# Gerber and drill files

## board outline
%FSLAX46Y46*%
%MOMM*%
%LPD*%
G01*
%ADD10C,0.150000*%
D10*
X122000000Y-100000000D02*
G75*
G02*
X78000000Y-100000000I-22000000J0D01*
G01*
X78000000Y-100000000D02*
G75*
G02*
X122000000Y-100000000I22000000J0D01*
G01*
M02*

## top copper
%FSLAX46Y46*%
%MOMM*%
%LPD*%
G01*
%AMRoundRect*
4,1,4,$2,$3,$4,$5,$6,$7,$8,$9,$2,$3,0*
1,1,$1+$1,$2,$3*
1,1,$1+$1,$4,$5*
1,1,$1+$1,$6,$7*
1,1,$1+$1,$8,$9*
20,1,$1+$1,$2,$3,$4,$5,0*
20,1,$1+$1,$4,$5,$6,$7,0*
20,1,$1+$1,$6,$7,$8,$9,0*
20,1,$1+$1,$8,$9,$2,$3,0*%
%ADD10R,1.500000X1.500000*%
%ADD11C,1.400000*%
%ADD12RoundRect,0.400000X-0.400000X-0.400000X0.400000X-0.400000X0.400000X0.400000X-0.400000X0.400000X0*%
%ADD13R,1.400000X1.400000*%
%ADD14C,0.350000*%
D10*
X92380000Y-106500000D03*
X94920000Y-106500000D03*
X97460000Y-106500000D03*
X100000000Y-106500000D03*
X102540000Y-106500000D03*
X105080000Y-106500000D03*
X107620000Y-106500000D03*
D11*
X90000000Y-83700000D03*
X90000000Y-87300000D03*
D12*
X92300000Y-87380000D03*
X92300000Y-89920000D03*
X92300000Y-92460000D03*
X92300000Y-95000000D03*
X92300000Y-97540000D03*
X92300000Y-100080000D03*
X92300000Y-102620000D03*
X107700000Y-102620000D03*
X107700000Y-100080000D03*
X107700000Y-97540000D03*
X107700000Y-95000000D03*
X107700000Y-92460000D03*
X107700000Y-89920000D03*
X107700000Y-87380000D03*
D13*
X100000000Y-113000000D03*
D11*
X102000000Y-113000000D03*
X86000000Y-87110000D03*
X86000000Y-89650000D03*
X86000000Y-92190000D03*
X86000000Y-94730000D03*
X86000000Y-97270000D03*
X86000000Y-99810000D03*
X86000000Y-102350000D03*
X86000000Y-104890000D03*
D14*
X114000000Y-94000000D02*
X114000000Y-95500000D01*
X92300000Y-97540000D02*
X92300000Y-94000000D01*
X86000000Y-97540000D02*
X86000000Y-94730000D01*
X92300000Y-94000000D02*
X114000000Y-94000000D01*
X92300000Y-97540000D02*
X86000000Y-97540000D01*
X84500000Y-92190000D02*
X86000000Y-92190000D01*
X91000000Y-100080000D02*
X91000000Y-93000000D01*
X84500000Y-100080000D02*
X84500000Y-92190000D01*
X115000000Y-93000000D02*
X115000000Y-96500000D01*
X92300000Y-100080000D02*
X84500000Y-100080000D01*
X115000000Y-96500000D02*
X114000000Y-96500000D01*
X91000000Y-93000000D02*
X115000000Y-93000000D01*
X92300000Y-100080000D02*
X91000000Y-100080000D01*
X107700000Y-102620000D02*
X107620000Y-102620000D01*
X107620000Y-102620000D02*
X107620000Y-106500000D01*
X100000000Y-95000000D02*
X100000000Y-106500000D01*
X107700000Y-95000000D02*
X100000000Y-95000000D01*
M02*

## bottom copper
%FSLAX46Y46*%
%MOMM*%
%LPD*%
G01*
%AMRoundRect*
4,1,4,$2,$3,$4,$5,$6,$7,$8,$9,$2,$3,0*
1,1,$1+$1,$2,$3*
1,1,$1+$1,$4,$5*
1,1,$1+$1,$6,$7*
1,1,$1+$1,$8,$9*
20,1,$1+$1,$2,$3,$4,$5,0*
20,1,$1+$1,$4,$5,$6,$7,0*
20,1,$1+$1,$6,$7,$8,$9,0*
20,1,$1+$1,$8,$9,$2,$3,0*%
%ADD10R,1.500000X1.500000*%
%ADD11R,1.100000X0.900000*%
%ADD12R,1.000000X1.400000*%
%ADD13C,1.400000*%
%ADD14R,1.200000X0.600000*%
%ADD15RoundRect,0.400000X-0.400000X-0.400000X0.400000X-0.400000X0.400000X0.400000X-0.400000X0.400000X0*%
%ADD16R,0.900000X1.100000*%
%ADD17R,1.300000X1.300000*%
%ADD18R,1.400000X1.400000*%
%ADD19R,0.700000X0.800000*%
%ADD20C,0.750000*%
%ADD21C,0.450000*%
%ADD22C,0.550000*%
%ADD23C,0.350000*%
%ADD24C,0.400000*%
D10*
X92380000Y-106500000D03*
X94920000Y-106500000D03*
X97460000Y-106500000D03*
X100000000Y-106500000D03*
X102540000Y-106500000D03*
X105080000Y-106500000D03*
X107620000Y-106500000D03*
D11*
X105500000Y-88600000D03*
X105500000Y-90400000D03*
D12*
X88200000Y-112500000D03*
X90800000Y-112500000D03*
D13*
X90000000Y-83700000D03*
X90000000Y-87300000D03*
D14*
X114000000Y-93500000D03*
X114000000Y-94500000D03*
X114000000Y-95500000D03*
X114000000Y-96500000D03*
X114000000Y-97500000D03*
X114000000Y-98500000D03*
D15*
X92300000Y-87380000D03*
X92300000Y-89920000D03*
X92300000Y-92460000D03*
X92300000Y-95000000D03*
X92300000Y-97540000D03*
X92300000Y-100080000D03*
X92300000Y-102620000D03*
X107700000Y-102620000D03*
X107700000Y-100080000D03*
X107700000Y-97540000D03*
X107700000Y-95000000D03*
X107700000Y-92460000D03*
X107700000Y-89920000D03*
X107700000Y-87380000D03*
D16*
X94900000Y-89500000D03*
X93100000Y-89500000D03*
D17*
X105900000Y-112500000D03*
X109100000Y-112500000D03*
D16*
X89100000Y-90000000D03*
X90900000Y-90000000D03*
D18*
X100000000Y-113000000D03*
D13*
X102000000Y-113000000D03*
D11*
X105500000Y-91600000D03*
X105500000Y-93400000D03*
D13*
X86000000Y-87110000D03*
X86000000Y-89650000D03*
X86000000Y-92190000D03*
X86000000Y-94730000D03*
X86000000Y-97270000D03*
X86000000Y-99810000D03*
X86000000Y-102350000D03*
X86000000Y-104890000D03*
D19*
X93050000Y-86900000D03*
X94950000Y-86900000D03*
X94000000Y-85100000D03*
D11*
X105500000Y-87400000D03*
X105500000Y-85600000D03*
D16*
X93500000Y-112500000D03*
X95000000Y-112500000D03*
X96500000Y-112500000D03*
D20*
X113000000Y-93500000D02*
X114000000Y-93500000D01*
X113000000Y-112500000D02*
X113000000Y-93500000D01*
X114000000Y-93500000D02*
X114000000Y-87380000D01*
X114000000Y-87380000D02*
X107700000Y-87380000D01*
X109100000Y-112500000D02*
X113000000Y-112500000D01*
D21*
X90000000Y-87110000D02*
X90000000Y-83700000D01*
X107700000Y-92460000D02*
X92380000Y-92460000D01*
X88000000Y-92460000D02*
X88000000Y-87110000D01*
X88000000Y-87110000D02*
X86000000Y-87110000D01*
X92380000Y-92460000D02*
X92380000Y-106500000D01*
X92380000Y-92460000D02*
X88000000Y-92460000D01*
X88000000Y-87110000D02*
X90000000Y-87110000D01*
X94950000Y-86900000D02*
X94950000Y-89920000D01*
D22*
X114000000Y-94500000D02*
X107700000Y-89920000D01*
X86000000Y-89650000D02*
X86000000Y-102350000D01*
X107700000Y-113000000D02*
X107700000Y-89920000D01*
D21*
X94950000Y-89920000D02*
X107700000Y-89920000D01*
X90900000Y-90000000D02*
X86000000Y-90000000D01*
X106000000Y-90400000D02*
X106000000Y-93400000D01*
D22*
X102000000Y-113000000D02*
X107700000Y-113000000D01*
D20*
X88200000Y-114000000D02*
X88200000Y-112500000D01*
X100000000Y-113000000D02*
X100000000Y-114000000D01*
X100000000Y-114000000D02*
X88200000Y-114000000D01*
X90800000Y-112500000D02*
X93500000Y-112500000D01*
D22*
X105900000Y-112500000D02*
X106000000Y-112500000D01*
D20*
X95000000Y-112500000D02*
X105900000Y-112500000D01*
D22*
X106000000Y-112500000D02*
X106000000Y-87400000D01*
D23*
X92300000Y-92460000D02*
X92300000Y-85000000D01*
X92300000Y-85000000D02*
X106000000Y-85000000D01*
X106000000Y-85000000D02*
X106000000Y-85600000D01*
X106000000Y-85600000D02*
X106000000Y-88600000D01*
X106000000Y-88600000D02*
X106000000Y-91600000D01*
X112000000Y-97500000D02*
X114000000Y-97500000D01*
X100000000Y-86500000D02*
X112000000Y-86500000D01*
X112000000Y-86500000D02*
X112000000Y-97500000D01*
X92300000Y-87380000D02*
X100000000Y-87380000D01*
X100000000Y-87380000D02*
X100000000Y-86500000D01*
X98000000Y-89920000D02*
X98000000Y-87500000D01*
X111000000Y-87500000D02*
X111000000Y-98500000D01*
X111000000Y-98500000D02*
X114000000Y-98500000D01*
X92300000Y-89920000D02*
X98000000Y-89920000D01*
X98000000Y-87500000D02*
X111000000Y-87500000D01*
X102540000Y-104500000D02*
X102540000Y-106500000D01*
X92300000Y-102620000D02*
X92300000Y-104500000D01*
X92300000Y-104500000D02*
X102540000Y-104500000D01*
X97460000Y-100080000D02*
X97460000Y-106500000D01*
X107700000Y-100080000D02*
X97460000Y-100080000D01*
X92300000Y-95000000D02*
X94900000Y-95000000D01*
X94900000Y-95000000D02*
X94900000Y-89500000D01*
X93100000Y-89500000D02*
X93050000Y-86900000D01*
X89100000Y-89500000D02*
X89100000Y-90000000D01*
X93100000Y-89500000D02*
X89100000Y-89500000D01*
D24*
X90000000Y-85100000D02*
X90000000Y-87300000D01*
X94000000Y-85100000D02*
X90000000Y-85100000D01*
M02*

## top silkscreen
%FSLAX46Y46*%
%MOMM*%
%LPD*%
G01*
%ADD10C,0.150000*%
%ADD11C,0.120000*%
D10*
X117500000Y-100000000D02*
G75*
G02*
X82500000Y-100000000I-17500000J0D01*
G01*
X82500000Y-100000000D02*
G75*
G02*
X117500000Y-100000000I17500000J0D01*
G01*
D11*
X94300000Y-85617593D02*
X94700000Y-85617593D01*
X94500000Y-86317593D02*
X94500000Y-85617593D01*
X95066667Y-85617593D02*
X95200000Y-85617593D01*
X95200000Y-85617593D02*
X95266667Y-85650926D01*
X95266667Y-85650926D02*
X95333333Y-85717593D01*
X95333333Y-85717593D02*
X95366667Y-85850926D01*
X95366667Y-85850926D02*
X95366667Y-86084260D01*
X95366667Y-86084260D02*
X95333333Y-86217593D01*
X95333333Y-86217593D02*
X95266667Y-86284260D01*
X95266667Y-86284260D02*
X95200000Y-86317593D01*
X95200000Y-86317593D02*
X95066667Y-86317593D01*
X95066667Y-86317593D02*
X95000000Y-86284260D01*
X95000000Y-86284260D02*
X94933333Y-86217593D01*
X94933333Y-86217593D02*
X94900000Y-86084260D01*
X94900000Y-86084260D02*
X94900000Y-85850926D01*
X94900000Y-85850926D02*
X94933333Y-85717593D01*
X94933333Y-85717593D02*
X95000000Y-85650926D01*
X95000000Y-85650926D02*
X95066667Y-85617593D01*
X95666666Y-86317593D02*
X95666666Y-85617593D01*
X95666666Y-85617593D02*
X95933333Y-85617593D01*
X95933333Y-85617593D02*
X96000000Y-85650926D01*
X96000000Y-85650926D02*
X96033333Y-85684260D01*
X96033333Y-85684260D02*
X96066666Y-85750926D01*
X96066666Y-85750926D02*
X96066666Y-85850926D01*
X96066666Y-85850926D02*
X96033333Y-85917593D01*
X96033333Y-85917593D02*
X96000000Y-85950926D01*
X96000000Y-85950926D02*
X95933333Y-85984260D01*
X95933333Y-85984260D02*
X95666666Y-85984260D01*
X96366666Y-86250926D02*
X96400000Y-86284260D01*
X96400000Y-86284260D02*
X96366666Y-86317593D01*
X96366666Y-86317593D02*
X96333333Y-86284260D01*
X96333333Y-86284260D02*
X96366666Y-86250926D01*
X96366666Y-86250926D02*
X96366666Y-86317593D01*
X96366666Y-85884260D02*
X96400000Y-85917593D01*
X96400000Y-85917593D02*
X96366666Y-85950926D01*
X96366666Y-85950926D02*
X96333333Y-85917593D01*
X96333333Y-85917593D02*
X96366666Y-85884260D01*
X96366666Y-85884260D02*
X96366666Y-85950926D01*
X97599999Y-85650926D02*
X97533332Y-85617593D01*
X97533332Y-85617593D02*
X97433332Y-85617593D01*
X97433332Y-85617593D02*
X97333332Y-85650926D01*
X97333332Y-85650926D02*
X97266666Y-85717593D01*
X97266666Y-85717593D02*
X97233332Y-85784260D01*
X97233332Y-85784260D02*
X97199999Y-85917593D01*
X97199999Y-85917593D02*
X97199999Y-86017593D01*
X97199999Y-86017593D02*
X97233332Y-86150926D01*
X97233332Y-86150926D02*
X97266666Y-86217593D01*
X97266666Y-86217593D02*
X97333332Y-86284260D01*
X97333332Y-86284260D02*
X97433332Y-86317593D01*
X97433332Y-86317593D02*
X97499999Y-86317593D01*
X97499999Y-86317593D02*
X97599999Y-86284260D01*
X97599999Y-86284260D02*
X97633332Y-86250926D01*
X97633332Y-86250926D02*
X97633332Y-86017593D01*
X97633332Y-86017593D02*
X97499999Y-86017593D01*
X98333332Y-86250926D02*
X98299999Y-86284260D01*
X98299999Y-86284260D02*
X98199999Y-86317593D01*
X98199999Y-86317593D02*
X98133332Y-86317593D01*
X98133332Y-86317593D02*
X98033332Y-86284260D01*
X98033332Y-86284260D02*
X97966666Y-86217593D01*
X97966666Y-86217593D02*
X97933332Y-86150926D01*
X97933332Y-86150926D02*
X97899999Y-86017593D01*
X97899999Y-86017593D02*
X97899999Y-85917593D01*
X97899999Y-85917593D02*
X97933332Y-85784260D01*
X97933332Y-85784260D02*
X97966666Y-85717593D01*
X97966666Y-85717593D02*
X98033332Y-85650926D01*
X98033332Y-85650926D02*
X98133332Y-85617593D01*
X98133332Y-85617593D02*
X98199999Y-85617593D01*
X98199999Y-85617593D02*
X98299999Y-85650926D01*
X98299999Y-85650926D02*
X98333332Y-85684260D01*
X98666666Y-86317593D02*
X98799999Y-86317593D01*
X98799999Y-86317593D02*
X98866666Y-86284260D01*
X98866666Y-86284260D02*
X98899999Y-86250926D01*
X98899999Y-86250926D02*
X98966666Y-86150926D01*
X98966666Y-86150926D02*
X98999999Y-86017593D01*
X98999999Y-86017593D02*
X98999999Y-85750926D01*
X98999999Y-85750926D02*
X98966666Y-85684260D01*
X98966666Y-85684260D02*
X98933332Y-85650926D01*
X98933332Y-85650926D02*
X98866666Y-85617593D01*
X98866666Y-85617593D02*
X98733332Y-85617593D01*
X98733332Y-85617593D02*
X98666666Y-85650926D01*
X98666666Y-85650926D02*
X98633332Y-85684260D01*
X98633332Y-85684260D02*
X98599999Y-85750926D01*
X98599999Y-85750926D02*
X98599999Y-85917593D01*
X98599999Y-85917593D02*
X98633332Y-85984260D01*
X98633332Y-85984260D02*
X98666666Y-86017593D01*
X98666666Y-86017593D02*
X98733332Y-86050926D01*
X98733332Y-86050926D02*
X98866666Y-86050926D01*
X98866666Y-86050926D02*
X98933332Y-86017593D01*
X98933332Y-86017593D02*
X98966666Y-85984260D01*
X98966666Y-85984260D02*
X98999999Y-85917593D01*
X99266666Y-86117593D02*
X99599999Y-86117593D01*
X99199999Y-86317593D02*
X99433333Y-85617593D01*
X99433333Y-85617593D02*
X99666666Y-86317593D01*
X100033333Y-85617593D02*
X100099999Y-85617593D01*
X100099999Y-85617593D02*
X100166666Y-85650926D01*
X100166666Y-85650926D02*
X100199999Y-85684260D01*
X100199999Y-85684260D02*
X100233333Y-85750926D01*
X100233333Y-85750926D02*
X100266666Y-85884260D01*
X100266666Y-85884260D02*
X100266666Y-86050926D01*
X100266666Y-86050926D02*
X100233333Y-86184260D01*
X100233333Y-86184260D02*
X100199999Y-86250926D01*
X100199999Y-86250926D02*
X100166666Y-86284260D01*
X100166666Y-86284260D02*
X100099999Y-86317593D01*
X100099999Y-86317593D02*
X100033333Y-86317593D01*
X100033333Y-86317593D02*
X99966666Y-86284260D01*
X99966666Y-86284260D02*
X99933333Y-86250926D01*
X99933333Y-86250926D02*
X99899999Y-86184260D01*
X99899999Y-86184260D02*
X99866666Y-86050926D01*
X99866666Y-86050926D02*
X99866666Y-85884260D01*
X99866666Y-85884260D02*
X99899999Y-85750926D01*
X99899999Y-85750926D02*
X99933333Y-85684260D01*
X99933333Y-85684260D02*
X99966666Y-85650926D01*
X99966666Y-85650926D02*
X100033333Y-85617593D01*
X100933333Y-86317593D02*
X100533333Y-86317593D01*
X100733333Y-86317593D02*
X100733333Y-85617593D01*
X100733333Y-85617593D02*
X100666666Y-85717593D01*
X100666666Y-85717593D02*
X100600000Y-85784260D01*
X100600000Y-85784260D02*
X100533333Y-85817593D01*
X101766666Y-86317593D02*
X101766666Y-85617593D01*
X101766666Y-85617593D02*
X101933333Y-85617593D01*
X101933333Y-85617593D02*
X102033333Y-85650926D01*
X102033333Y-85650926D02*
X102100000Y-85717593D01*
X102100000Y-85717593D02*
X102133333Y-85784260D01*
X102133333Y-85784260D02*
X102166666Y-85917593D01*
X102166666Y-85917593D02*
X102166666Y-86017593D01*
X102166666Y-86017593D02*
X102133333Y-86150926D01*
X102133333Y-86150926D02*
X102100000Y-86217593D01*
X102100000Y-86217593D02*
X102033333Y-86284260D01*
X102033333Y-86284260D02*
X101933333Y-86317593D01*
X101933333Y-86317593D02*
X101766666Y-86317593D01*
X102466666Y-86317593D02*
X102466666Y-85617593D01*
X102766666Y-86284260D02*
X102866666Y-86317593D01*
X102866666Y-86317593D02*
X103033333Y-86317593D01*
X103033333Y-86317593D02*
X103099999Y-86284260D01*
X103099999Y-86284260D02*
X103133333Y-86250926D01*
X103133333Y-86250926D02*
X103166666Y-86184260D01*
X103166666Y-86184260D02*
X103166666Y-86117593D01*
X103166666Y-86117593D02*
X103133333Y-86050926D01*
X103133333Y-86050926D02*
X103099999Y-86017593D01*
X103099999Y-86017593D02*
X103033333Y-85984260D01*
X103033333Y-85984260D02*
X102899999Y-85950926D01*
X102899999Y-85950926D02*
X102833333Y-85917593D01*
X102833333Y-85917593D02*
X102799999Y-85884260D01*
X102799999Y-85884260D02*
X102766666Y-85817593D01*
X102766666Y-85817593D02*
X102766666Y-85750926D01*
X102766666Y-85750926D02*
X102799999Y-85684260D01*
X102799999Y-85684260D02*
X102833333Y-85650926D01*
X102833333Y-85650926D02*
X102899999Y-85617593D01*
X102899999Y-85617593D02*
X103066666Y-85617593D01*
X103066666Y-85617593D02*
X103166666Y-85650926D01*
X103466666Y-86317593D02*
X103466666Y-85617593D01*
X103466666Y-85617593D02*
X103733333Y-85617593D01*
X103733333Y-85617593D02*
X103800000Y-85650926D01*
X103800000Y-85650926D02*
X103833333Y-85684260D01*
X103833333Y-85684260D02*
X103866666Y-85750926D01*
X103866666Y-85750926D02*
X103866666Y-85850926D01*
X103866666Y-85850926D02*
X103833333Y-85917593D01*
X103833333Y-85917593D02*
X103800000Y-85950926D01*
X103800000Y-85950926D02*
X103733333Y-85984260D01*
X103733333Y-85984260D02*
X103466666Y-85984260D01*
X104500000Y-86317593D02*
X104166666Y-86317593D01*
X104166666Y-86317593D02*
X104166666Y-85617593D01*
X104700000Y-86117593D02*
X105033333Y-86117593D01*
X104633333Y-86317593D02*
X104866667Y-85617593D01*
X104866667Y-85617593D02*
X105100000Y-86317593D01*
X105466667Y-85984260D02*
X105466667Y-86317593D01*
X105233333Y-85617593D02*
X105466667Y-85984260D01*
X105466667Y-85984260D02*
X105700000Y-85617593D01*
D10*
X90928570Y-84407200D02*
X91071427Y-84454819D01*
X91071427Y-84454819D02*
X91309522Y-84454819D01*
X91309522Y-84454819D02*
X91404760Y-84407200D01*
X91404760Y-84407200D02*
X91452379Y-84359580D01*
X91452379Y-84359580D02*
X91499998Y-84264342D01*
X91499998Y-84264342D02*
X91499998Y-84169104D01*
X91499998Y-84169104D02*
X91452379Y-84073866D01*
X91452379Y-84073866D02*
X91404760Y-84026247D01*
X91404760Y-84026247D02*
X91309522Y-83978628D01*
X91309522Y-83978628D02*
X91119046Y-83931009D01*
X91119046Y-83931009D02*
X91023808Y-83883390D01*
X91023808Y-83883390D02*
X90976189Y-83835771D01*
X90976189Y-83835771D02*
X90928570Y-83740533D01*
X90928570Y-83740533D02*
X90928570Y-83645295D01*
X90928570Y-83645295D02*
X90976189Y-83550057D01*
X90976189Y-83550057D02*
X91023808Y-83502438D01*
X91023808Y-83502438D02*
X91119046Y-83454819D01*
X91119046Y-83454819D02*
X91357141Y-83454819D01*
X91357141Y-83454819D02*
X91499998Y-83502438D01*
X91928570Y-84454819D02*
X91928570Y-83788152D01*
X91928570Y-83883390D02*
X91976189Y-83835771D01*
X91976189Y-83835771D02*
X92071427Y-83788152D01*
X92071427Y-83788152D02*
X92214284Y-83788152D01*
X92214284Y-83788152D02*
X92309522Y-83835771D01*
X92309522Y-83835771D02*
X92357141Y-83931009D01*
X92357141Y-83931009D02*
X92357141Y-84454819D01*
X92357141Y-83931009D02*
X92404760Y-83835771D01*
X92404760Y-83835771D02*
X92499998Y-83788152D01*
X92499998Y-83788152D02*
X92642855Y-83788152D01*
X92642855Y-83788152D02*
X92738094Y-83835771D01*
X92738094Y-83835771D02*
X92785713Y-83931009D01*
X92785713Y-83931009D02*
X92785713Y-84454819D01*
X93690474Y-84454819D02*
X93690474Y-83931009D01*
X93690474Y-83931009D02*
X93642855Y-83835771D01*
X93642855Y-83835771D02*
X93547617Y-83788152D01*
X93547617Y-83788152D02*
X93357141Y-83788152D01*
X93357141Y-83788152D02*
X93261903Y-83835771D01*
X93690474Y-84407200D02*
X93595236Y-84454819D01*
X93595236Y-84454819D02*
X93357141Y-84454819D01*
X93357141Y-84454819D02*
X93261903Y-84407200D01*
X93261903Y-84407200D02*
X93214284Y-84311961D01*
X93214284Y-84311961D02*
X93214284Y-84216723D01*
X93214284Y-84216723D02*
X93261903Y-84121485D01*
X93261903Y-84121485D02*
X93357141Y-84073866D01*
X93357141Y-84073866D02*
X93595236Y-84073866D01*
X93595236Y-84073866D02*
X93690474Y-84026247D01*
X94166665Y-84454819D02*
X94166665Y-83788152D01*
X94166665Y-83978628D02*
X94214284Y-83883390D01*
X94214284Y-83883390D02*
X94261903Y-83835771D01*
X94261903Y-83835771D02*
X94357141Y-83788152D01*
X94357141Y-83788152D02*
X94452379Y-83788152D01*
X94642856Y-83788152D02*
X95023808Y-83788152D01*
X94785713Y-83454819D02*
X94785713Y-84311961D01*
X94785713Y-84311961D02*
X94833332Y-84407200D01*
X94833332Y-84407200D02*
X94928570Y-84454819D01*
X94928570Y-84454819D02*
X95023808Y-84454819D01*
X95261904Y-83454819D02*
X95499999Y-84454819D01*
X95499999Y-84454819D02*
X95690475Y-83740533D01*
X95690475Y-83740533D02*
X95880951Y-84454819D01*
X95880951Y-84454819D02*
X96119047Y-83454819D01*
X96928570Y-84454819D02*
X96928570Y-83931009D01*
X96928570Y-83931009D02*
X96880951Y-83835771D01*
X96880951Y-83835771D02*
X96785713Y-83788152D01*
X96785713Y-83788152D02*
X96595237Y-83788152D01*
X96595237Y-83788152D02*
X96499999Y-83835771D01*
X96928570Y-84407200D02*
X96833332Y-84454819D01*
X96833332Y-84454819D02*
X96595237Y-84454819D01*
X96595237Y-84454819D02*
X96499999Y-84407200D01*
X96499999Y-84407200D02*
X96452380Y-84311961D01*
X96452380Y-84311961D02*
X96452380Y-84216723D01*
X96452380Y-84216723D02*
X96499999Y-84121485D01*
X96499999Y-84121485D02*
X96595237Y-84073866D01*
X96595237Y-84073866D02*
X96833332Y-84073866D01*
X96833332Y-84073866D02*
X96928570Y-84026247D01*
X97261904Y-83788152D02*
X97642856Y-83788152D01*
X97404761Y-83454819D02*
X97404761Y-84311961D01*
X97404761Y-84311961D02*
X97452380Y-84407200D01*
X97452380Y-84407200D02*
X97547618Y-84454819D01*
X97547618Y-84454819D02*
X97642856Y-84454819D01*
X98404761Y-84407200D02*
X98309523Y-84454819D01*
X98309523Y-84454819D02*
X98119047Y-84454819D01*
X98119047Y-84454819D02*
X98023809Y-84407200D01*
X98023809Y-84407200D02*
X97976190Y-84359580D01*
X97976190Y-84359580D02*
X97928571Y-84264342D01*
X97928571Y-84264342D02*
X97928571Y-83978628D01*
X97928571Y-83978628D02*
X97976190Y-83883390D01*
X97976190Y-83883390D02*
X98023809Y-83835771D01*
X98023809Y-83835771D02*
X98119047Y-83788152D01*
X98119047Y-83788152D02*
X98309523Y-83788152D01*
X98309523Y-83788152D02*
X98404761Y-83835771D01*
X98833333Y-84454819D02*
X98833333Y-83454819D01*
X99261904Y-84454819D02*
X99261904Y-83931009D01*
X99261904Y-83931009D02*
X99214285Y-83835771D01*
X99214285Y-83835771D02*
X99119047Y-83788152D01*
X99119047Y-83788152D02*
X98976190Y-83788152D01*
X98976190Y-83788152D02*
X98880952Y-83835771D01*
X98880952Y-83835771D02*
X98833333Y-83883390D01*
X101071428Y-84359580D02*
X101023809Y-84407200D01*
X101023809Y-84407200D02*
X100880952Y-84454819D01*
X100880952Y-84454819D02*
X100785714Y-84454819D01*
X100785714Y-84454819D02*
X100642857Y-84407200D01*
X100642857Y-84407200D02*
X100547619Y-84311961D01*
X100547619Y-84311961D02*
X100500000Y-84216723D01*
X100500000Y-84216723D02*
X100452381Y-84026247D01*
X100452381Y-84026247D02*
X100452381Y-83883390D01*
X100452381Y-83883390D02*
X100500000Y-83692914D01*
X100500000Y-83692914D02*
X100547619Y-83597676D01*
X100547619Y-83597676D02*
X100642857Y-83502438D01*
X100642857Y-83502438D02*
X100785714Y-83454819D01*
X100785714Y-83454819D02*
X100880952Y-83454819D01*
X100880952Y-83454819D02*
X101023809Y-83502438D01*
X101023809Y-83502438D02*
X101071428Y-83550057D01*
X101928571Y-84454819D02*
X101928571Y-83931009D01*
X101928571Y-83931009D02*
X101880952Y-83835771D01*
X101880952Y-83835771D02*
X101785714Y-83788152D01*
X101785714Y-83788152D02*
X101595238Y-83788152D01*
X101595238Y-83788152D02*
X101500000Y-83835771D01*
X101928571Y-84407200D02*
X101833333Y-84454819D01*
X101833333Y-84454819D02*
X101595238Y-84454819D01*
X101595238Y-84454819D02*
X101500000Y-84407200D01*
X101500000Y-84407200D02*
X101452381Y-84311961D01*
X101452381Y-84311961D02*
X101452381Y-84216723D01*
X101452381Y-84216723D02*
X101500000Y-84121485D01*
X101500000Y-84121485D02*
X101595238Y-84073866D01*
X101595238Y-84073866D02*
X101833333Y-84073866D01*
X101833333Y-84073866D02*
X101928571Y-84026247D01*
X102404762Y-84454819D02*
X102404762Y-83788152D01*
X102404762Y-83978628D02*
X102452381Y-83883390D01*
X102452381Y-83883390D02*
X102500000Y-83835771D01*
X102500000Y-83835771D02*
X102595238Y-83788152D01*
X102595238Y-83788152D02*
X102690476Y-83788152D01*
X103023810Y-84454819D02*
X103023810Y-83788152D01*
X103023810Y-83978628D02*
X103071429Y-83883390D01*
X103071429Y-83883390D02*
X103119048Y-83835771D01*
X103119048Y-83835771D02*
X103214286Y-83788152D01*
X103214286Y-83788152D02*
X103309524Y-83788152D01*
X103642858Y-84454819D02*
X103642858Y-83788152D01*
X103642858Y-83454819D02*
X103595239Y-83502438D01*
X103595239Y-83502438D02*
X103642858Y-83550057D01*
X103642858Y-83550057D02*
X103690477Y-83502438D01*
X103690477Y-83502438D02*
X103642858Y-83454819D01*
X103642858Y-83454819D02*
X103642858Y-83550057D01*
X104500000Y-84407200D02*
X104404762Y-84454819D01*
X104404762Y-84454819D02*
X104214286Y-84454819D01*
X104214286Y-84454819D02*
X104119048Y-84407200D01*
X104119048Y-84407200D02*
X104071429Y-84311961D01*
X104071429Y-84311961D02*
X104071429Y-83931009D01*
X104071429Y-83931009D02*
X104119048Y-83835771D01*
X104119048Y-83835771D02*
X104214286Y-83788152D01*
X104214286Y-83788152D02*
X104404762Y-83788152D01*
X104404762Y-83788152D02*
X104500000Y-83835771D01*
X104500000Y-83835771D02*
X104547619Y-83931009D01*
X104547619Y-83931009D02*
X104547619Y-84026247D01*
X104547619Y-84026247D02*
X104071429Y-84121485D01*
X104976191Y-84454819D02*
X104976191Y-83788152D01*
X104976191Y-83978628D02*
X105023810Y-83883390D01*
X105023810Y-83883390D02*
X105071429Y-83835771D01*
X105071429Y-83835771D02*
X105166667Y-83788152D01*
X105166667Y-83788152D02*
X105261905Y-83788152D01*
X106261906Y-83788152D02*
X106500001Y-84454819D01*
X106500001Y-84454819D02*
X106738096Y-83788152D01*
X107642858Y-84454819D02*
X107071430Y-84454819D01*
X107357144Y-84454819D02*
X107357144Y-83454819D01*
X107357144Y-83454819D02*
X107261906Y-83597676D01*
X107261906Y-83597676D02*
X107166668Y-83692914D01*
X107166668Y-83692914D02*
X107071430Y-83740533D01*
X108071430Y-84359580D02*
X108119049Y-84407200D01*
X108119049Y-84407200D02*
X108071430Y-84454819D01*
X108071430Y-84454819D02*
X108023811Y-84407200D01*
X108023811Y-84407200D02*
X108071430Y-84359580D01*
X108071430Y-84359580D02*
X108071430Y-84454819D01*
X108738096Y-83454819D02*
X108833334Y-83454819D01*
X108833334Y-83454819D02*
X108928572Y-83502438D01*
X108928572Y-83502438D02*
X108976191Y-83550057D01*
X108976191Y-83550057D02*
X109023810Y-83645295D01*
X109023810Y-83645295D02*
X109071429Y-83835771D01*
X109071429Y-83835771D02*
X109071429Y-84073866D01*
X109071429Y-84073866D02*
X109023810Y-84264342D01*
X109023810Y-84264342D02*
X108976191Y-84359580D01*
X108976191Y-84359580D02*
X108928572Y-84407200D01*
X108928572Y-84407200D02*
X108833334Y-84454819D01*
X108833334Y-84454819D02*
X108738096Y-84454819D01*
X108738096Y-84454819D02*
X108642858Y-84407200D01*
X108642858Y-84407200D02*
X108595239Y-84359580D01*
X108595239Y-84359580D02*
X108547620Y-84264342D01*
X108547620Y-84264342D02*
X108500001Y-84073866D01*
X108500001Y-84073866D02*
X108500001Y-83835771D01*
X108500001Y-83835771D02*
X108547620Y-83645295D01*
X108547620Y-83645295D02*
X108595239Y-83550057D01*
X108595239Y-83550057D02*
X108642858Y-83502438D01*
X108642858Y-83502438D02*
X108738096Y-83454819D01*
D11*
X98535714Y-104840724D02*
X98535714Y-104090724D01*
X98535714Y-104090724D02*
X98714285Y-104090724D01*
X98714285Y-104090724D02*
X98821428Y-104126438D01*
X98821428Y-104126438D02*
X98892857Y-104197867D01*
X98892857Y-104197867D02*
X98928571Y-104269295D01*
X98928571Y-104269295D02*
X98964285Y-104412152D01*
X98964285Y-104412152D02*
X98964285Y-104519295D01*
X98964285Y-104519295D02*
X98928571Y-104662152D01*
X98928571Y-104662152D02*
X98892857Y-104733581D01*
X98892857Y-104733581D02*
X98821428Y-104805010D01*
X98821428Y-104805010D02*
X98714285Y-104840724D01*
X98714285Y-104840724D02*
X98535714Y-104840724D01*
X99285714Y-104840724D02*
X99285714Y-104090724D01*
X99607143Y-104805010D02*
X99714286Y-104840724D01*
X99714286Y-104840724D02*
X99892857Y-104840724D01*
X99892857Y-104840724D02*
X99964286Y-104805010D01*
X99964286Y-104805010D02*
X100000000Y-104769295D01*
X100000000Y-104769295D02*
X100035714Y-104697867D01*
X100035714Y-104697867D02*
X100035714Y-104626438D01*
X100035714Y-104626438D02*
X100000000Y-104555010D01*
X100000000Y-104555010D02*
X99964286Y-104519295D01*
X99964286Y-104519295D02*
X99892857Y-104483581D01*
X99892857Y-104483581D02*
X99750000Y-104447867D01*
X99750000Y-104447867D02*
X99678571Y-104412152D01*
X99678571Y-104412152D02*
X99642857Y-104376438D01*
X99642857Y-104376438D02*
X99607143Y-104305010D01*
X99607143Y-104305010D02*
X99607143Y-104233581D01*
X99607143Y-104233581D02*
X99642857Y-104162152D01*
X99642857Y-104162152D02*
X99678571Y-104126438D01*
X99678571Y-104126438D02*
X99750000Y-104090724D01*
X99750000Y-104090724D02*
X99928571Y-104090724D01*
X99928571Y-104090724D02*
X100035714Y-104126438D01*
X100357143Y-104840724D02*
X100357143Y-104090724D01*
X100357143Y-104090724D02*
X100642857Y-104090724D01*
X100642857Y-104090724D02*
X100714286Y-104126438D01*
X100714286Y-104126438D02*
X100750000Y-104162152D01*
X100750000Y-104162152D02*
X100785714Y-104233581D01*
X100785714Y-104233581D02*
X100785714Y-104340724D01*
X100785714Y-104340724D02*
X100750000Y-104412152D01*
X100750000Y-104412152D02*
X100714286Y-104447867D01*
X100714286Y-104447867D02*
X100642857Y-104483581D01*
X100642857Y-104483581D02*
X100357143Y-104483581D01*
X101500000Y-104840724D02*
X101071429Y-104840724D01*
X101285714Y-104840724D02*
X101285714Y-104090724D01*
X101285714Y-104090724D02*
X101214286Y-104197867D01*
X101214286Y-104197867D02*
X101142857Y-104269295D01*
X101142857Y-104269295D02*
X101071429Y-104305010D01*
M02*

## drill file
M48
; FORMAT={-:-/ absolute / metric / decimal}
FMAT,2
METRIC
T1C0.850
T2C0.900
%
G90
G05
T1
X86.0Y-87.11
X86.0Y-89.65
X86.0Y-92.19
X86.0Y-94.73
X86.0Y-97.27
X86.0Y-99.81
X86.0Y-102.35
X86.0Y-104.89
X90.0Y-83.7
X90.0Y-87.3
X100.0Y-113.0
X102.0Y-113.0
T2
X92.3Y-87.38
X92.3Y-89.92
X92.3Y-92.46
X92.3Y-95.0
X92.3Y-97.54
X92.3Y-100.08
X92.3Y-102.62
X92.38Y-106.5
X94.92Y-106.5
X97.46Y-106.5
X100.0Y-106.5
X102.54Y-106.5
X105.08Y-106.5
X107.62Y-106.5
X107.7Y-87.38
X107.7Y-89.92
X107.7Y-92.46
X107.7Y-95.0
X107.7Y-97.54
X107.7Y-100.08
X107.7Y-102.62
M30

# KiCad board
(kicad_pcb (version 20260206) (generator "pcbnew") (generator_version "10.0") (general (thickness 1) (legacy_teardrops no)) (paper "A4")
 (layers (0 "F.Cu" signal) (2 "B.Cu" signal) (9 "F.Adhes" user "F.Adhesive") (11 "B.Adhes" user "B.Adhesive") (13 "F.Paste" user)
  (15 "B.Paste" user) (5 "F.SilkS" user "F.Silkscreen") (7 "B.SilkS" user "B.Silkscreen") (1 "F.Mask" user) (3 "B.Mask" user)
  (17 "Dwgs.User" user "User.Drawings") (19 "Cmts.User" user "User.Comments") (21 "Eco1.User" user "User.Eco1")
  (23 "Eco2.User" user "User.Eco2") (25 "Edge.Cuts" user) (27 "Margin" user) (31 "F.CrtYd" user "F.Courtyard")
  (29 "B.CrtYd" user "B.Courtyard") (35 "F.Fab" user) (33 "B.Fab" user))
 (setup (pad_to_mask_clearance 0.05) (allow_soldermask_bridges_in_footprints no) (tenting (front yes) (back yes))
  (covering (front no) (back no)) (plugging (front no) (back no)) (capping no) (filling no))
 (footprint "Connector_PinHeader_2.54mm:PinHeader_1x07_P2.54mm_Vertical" (layer "F.Cu") (at 100 106.5)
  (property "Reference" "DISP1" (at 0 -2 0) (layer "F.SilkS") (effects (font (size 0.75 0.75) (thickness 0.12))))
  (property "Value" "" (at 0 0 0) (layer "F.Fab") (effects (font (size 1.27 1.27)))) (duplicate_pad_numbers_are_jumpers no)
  (pad "1" thru_hole rect (at -7.62 0) (size 1.5 1.5) (drill 0.9) (layers "*.Cu" "*.Mask") (remove_unused_layers no) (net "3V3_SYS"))
  (pad "2" thru_hole rect (at -5.08 0) (size 1.5 1.5) (drill 0.9) (layers "*.Cu" "*.Mask") (remove_unused_layers no) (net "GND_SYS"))
  (pad "3" thru_hole rect (at -2.54 0) (size 1.5 1.5) (drill 0.9) (layers "*.Cu" "*.Mask") (remove_unused_layers no) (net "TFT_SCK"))
  (pad "4" thru_hole rect (at 0 0) (size 1.5 1.5) (drill 0.9) (layers "*.Cu" "*.Mask") (remove_unused_layers no) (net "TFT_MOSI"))
  (pad "5" thru_hole rect (at 2.54 0) (size 1.5 1.5) (drill 0.9) (layers "*.Cu" "*.Mask") (remove_unused_layers no) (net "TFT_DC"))
  (pad "6" thru_hole rect (at 5.08 0) (size 1.5 1.5) (drill 0.9) (layers "*.Cu" "*.Mask") (remove_unused_layers no) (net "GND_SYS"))
  (pad "7" thru_hole rect (at 7.62 0) (size 1.5 1.5) (drill 0.9) (layers "*.Cu" "*.Mask") (remove_unused_layers no) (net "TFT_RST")))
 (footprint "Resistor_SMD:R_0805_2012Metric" (layer "B.Cu") (at 105.5 89.5)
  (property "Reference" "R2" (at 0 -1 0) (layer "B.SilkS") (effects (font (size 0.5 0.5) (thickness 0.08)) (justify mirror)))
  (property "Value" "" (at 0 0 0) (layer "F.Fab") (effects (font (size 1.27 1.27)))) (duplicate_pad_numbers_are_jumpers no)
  (pad "1" smd rect (at 0 -0.9) (size 1.1 0.9) (layers "B.Cu" "B.Mask" "B.Paste") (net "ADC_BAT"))
  (pad "2" smd rect (at 0 0.9) (size 1.1 0.9) (layers "B.Cu" "B.Mask" "B.Paste") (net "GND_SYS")))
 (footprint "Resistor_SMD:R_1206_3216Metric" (layer "B.Cu") (at 89.5 112.5)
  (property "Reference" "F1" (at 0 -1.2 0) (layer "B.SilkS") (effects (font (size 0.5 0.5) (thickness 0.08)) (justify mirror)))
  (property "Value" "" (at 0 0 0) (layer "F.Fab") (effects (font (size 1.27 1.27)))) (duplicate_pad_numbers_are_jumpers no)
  (pad "1" smd rect (at -1.3 0) (size 1 1.4) (layers "B.Cu" "B.Mask" "B.Paste") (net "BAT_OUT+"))
  (pad "2" smd rect (at 1.3 0) (size 1 1.4) (layers "B.Cu" "B.Mask" "B.Paste") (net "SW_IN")))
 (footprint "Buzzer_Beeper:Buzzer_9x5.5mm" (layer "B.Cu") (at 90 85.5)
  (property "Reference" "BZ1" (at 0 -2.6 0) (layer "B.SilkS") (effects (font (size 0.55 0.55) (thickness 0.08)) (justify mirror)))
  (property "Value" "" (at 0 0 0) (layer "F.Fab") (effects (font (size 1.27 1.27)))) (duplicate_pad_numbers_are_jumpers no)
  (pad "1" thru_hole circle (at 0 -1.8) (size 1.4 1.4) (drill 0.85) (layers "*.Cu" "*.Mask") (remove_unused_layers no) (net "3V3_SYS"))
  (pad "2" thru_hole circle (at 0 1.8) (size 1.4 1.4) (drill 0.85) (layers "*.Cu" "*.Mask") (remove_unused_layers no) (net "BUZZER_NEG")))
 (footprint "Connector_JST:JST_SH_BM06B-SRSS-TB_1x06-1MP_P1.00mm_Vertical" (layer "B.Cu") (at 114 96)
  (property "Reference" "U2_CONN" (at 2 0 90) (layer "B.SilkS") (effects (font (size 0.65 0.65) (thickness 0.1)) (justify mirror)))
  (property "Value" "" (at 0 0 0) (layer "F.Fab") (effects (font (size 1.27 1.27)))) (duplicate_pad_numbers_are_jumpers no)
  (pad "1" smd rect (at 0 -2.5) (size 1.2 0.6) (layers "B.Cu" "B.Mask" "B.Paste") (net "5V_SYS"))
  (pad "2" smd rect (at 0 -1.5) (size 1.2 0.6) (layers "B.Cu" "B.Mask" "B.Paste") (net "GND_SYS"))
  (pad "3" smd rect (at 0 -0.5) (size 1.2 0.6) (layers "B.Cu" "B.Mask" "B.Paste") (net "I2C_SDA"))
  (pad "4" smd rect (at 0 0.5) (size 1.2 0.6) (layers "B.Cu" "B.Mask" "B.Paste") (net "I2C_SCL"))
  (pad "5" smd rect (at 0 1.5) (size 1.2 0.6) (layers "B.Cu" "B.Mask" "B.Paste") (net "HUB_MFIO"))
  (pad "6" smd rect (at 0 2.5) (size 1.2 0.6) (layers "B.Cu" "B.Mask" "B.Paste") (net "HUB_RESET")))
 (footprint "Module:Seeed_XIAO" (layer "B.Cu") (at 100 95)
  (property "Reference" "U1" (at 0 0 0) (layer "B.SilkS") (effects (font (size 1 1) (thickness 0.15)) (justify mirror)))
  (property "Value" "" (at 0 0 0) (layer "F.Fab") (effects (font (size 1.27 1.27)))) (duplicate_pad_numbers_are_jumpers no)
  (pad "1" thru_hole roundrect (at -7.7 -7.62) (size 1.6 1.6) (drill 0.9) (layers "*.Cu" "*.Mask") (remove_unused_layers no)
   (roundrect_rratio 0.25) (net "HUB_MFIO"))
  (pad "2" thru_hole roundrect (at -7.7 -5.08) (size 1.6 1.6) (drill 0.9) (layers "*.Cu" "*.Mask") (remove_unused_layers no)
   (roundrect_rratio 0.25) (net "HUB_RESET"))
  (pad "3" thru_hole roundrect (at -7.7 -2.54) (size 1.6 1.6) (drill 0.9) (layers "*.Cu" "*.Mask") (remove_unused_layers no)
   (roundrect_rratio 0.25) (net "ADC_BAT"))
  (pad "4" thru_hole roundrect (at -7.7 0) (size 1.6 1.6) (drill 0.9) (layers "*.Cu" "*.Mask") (remove_unused_layers no)
   (roundrect_rratio 0.25) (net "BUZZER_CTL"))
  (pad "5" thru_hole roundrect (at -7.7 2.54) (size 1.6 1.6) (drill 0.9) (layers "*.Cu" "*.Mask") (remove_unused_layers no)
   (roundrect_rratio 0.25) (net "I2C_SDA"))
  (pad "6" thru_hole roundrect (at -7.7 5.08) (size 1.6 1.6) (drill 0.9) (layers "*.Cu" "*.Mask") (remove_unused_layers no)
   (roundrect_rratio 0.25) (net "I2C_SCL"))
  (pad "7" thru_hole roundrect (at -7.7 7.62) (size 1.6 1.6) (drill 0.9) (layers "*.Cu" "*.Mask") (remove_unused_layers no)
   (roundrect_rratio 0.25) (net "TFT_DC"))
  (pad "8" thru_hole roundrect (at 7.7 7.62) (size 1.6 1.6) (drill 0.9) (layers "*.Cu" "*.Mask") (remove_unused_layers no)
   (roundrect_rratio 0.25) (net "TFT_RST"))
  (pad "9" thru_hole roundrect (at 7.7 5.08) (size 1.6 1.6) (drill 0.9) (layers "*.Cu" "*.Mask") (remove_unused_layers no)
   (roundrect_rratio 0.25) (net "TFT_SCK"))
  (pad "10" thru_hole roundrect (at 7.7 2.54) (size 1.6 1.6) (drill 0.9) (layers "*.Cu" "*.Mask") (remove_unused_layers no)
   (roundrect_rratio 0.25))
  (pad "11" thru_hole roundrect (at 7.7 0) (size 1.6 1.6) (drill 0.9) (layers "*.Cu" "*.Mask") (remove_unused_layers no)
   (roundrect_rratio 0.25) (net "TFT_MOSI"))
  (pad "12" thru_hole roundrect (at 7.7 -2.54) (size 1.6 1.6) (drill 0.9) (layers "*.Cu" "*.Mask") (remove_unused_layers no)
   (roundrect_rratio 0.25) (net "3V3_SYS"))
  (pad "13" thru_hole roundrect (at 7.7 -5.08) (size 1.6 1.6) (drill 0.9) (layers "*.Cu" "*.Mask") (remove_unused_layers no)
   (roundrect_rratio 0.25) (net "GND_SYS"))
  (pad "14" thru_hole roundrect (at 7.7 -7.62) (size 1.6 1.6) (drill 0.9) (layers "*.Cu" "*.Mask") (remove_unused_layers no)
   (roundrect_rratio 0.25) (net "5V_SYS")))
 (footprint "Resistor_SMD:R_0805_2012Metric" (layer "B.Cu") (at 94 89.5)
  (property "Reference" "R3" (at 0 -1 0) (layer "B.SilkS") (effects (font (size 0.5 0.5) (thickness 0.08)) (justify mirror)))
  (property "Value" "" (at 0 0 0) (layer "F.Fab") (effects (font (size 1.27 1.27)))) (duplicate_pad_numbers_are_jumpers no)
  (pad "1" smd rect (at 0.9 0) (size 0.9 1.1) (layers "B.Cu" "B.Mask" "B.Paste") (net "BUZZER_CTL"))
  (pad "2" smd rect (at -0.9 0) (size 0.9 1.1) (layers "B.Cu" "B.Mask" "B.Paste") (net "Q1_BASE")))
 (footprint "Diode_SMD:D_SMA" (layer "B.Cu") (at 107.5 112.5)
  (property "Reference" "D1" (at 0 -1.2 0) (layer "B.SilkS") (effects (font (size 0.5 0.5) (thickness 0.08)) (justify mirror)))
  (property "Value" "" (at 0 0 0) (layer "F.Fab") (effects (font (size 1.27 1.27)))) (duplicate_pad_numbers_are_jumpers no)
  (pad "1" smd rect (at -1.6 0) (size 1.3 1.3) (layers "B.Cu" "B.Mask" "B.Paste") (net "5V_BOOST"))
  (pad "2" smd rect (at 1.6 0) (size 1.3 1.3) (layers "B.Cu" "B.Mask" "B.Paste") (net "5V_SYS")))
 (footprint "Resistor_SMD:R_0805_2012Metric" (layer "B.Cu") (at 90 90)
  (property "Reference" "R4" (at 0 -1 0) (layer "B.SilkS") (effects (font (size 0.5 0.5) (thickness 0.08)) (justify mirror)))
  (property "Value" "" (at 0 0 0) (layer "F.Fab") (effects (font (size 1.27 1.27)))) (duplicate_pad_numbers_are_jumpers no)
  (pad "1" smd rect (at -0.9 0) (size 0.9 1.1) (layers "B.Cu" "B.Mask" "B.Paste") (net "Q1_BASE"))
  (pad "2" smd rect (at 0.9 0) (size 0.9 1.1) (layers "B.Cu" "B.Mask" "B.Paste") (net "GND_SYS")))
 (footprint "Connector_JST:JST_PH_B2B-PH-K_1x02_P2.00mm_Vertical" (layer "B.Cu") (at 101 113)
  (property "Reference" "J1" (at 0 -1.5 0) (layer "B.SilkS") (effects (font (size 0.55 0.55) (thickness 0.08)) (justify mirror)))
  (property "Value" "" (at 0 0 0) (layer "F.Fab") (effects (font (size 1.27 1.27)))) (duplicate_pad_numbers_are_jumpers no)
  (pad "1" thru_hole rect (at -1 0) (size 1.4 1.4) (drill 0.85) (layers "*.Cu" "*.Mask") (remove_unused_layers no) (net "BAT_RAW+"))
  (pad "2" thru_hole circle (at 1 0) (size 1.4 1.4) (drill 0.85) (layers "*.Cu" "*.Mask") (remove_unused_layers no) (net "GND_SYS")))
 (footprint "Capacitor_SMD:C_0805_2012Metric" (layer "B.Cu") (at 105.5 92.5)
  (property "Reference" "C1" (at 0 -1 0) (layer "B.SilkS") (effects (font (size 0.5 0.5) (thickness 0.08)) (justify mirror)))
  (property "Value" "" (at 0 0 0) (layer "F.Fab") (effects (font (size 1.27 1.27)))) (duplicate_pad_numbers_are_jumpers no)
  (pad "1" smd rect (at 0 -0.9) (size 1.1 0.9) (layers "B.Cu" "B.Mask" "B.Paste") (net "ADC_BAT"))
  (pad "2" smd rect (at 0 0.9) (size 1.1 0.9) (layers "B.Cu" "B.Mask" "B.Paste") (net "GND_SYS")))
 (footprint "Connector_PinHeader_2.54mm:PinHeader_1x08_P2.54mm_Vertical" (layer "B.Cu") (at 86 96)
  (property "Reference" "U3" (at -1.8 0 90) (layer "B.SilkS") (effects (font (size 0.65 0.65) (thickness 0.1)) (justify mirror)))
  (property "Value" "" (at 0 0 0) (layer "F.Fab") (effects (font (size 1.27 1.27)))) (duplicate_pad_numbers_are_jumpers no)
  (pad "1" thru_hole circle (at 0 -8.89) (size 1.4 1.4) (drill 0.85) (layers "*.Cu" "*.Mask") (remove_unused_layers no) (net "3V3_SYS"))
  (pad "2" thru_hole circle (at 0 -6.35) (size 1.4 1.4) (drill 0.85) (layers "*.Cu" "*.Mask") (remove_unused_layers no) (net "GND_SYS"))
  (pad "3" thru_hole circle (at 0 -3.81) (size 1.4 1.4) (drill 0.85) (layers "*.Cu" "*.Mask") (remove_unused_layers no) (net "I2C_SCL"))
  (pad "4" thru_hole circle (at 0 -1.27) (size 1.4 1.4) (drill 0.85) (layers "*.Cu" "*.Mask") (remove_unused_layers no) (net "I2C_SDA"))
  (pad "5" thru_hole circle (at 0 1.27) (size 1.4 1.4) (drill 0.85) (layers "*.Cu" "*.Mask") (remove_unused_layers no))
  (pad "6" thru_hole circle (at 0 3.81) (size 1.4 1.4) (drill 0.85) (layers "*.Cu" "*.Mask") (remove_unused_layers no))
  (pad "7" thru_hole circle (at 0 6.35) (size 1.4 1.4) (drill 0.85) (layers "*.Cu" "*.Mask") (remove_unused_layers no) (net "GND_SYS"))
  (pad "8" thru_hole circle (at 0 8.89) (size 1.4 1.4) (drill 0.85) (layers "*.Cu" "*.Mask") (remove_unused_layers no)))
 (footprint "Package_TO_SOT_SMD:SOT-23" (layer "B.Cu") (at 94 86)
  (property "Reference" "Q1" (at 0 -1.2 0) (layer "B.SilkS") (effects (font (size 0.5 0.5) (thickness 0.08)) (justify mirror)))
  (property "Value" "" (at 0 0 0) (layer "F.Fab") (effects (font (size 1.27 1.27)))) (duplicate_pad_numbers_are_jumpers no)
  (pad "1" smd rect (at -0.95 0.9) (size 0.7 0.8) (layers "B.Cu" "B.Mask" "B.Paste") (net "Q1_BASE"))
  (pad "2" smd rect (at 0.95 0.9) (size 0.7 0.8) (layers "B.Cu" "B.Mask" "B.Paste") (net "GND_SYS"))
  (pad "3" smd rect (at 0 -0.9) (size 0.7 0.8) (layers "B.Cu" "B.Mask" "B.Paste") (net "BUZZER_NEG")))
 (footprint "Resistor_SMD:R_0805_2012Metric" (layer "B.Cu") (at 105.5 86.5)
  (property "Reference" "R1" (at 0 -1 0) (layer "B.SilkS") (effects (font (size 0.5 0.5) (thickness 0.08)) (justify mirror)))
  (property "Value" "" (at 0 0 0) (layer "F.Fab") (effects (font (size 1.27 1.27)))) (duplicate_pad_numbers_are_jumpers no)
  (pad "1" smd rect (at 0 0.9) (size 1.1 0.9) (layers "B.Cu" "B.Mask" "B.Paste") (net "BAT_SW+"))
  (pad "2" smd rect (at 0 -0.9) (size 1.1 0.9) (layers "B.Cu" "B.Mask" "B.Paste") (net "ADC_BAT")))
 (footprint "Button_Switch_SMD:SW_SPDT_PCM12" (layer "B.Cu") (at 95 112.5)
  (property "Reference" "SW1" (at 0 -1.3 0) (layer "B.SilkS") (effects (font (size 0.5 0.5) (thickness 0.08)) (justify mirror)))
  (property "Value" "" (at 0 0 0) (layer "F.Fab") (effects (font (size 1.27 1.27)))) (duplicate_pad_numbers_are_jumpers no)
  (pad "1" smd rect (at -1.5 0) (size 0.9 1.1) (layers "B.Cu" "B.Mask" "B.Paste") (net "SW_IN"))
  (pad "2" smd rect (at 0 0) (size 0.9 1.1) (layers "B.Cu" "B.Mask" "B.Paste") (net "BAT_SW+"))
  (pad "3" smd rect (at 1.5 0) (size 0.9 1.1) (layers "B.Cu" "B.Mask" "B.Paste")))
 (gr_circle (center 100 100) (end 117.5 100) (stroke (width 0.15) (type solid)) (fill no) (layer "F.SilkS"))
 (gr_circle (center 100 100) (end 122 100) (stroke (width 0.15) (type solid)) (fill no) (layer "Edge.Cuts"))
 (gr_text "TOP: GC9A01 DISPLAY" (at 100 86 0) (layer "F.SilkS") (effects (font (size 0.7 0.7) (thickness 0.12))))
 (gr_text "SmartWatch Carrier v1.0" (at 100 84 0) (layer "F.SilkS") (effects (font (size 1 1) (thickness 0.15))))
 (segment (start 113 93.5) (end 114 93.5) (width 0.75) (layer "B.Cu") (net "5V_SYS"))
 (segment (start 113 112.5) (end 113 93.5) (width 0.75) (layer "B.Cu") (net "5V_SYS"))
 (segment (start 114 93.5) (end 114 87.38) (width 0.75) (layer "B.Cu") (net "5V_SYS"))
 (segment (start 114 87.38) (end 107.7 87.38) (width 0.75) (layer "B.Cu") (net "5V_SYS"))
 (segment (start 109.1 112.5) (end 113 112.5) (width 0.75) (layer "B.Cu") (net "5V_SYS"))
 (segment (start 90 87.11) (end 90 83.7) (width 0.45) (layer "B.Cu") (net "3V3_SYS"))
 (segment (start 107.7 92.46) (end 92.38 92.46) (width 0.45) (layer "B.Cu") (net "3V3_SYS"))
 (segment (start 88 92.46) (end 88 87.11) (width 0.45) (layer "B.Cu") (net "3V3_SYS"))
 (segment (start 88 87.11) (end 86 87.11) (width 0.45) (layer "B.Cu") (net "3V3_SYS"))
 (segment (start 92.38 92.46) (end 92.38 106.5) (width 0.45) (layer "B.Cu") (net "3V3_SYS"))
 (segment (start 92.38 92.46) (end 88 92.46) (width 0.45) (layer "B.Cu") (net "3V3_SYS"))
 (segment (start 88 87.11) (end 90 87.11) (width 0.45) (layer "B.Cu") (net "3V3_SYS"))
 (segment (start 94.95 86.9) (end 94.95 89.92) (width 0.45) (layer "B.Cu") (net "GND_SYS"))
 (segment (start 114 94.5) (end 107.7 89.92) (width 0.55) (layer "B.Cu") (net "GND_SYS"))
 (segment (start 86 89.65) (end 86 102.35) (width 0.55) (layer "B.Cu") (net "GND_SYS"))
 (segment (start 107.7 113) (end 107.7 89.92) (width 0.55) (layer "B.Cu") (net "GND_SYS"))
 (segment (start 94.95 89.92) (end 107.7 89.92) (width 0.45) (layer "B.Cu") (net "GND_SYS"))
 (segment (start 90.9 90) (end 86 90) (width 0.45) (layer "B.Cu") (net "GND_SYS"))
 (segment (start 106 90.4) (end 106 93.4) (width 0.45) (layer "B.Cu") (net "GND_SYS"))
 (segment (start 102 113) (end 107.7 113) (width 0.55) (layer "B.Cu") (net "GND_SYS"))
 (segment (start 88.2 114) (end 88.2 112.5) (width 0.75) (layer "B.Cu") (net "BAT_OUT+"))
 (segment (start 100 113) (end 100 114) (width 0.75) (layer "B.Cu") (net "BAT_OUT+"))
 (segment (start 100 114) (end 88.2 114) (width 0.75) (layer "B.Cu") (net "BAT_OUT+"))
 (segment (start 90.8 112.5) (end 93.5 112.5) (width 0.75) (layer "B.Cu") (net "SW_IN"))
 (segment (start 105.9 112.5) (end 106 112.5) (width 0.55) (layer "B.Cu") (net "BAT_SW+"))
 (segment (start 95 112.5) (end 105.9 112.5) (width 0.75) (layer "B.Cu") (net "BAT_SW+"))
 (segment (start 106 112.5) (end 106 87.4) (width 0.55) (layer "B.Cu") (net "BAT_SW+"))
 (segment (start 92.3 92.46) (end 92.3 85) (width 0.35) (layer "B.Cu") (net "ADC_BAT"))
 (segment (start 92.3 85) (end 106 85) (width 0.35) (layer "B.Cu") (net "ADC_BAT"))
 (segment (start 106 85) (end 106 85.6) (width 0.35) (layer "B.Cu") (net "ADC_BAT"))
 (segment (start 106 85.6) (end 106 88.6) (width 0.35) (layer "B.Cu") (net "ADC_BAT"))
 (segment (start 106 88.6) (end 106 91.6) (width 0.35) (layer "B.Cu") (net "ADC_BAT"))
 (segment (start 112 97.5) (end 114 97.5) (width 0.35) (layer "B.Cu") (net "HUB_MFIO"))
 (segment (start 100 86.5) (end 112 86.5) (width 0.35) (layer "B.Cu") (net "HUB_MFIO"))
 (segment (start 112 86.5) (end 112 97.5) (width 0.35) (layer "B.Cu") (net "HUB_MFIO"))
 (segment (start 92.3 87.38) (end 100 87.38) (width 0.35) (layer "B.Cu") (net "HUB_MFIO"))
 (segment (start 100 87.38) (end 100 86.5) (width 0.35) (layer "B.Cu") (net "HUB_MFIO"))
 (segment (start 98 89.92) (end 98 87.5) (width 0.35) (layer "B.Cu") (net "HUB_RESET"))
 (segment (start 111 87.5) (end 111 98.5) (width 0.35) (layer "B.Cu") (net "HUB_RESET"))
 (segment (start 111 98.5) (end 114 98.5) (width 0.35) (layer "B.Cu") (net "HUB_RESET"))
 (segment (start 92.3 89.92) (end 98 89.92) (width 0.35) (layer "B.Cu") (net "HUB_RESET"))
 (segment (start 98 87.5) (end 111 87.5) (width 0.35) (layer "B.Cu") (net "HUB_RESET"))
 (segment (start 114 94) (end 114 95.5) (width 0.35) (layer "F.Cu") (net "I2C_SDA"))
 (segment (start 92.3 97.54) (end 92.3 94) (width 0.35) (layer "F.Cu") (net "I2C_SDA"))
 (segment (start 86 97.54) (end 86 94.73) (width 0.35) (layer "F.Cu") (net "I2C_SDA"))
 (segment (start 92.3 94) (end 114 94) (width 0.35) (layer "F.Cu") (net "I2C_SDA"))
 (segment (start 92.3 97.54) (end 86 97.54) (width 0.35) (layer "F.Cu") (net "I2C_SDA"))
 (segment (start 84.5 92.19) (end 86 92.19) (width 0.35) (layer "F.Cu") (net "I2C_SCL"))
 (segment (start 91 100.08) (end 91 93) (width 0.35) (layer "F.Cu") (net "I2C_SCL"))
 (segment (start 84.5 100.08) (end 84.5 92.19) (width 0.35) (layer "F.Cu") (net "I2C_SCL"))
 (segment (start 115 93) (end 115 96.5) (width 0.35) (layer "F.Cu") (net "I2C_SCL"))
 (segment (start 92.3 100.08) (end 84.5 100.08) (width 0.35) (layer "F.Cu") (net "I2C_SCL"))
 (segment (start 115 96.5) (end 114 96.5) (width 0.35) (layer "F.Cu") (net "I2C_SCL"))
 (segment (start 91 93) (end 115 93) (width 0.35) (layer "F.Cu") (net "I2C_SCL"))
 (segment (start 92.3 100.08) (end 91 100.08) (width 0.35) (layer "F.Cu") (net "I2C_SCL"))
 (segment (start 102.54 104.5) (end 102.54 106.5) (width 0.35) (layer "B.Cu") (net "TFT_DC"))
 (segment (start 92.3 102.62) (end 92.3 104.5) (width 0.35) (layer "B.Cu") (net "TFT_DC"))
 (segment (start 92.3 104.5) (end 102.54 104.5) (width 0.35) (layer "B.Cu") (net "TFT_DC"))
 (segment (start 107.7 102.62) (end 107.62 102.62) (width 0.35) (layer "F.Cu") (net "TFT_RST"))
 (segment (start 107.62 102.62) (end 107.62 106.5) (width 0.35) (layer "F.Cu") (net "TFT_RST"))
 (segment (start 97.46 100.08) (end 97.46 106.5) (width 0.35) (layer "B.Cu") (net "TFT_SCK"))
 (segment (start 107.7 100.08) (end 97.46 100.08) (width 0.35) (layer "B.Cu") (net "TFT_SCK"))
 (segment (start 100 95) (end 100 106.5) (width 0.35) (layer "F.Cu") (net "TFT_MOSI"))
 (segment (start 107.7 95) (end 100 95) (width 0.35) (layer "F.Cu") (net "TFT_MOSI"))
 (segment (start 92.3 95) (end 94.9 95) (width 0.35) (layer "B.Cu") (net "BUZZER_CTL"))
 (segment (start 94.9 95) (end 94.9 89.5) (width 0.35) (layer "B.Cu") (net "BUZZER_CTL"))
 (segment (start 93.1 89.5) (end 93.05 86.9) (width 0.35) (layer "B.Cu") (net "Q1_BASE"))
 (segment (start 89.1 89.5) (end 89.1 90) (width 0.35) (layer "B.Cu") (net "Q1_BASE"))
 (segment (start 93.1 89.5) (end 89.1 89.5) (width 0.35) (layer "B.Cu") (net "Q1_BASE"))
 (segment (start 90 85.1) (end 90 87.3) (width 0.4) (layer "B.Cu") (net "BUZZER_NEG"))
 (segment (start 94 85.1) (end 90 85.1) (width 0.4) (layer "B.Cu") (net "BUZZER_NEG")))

